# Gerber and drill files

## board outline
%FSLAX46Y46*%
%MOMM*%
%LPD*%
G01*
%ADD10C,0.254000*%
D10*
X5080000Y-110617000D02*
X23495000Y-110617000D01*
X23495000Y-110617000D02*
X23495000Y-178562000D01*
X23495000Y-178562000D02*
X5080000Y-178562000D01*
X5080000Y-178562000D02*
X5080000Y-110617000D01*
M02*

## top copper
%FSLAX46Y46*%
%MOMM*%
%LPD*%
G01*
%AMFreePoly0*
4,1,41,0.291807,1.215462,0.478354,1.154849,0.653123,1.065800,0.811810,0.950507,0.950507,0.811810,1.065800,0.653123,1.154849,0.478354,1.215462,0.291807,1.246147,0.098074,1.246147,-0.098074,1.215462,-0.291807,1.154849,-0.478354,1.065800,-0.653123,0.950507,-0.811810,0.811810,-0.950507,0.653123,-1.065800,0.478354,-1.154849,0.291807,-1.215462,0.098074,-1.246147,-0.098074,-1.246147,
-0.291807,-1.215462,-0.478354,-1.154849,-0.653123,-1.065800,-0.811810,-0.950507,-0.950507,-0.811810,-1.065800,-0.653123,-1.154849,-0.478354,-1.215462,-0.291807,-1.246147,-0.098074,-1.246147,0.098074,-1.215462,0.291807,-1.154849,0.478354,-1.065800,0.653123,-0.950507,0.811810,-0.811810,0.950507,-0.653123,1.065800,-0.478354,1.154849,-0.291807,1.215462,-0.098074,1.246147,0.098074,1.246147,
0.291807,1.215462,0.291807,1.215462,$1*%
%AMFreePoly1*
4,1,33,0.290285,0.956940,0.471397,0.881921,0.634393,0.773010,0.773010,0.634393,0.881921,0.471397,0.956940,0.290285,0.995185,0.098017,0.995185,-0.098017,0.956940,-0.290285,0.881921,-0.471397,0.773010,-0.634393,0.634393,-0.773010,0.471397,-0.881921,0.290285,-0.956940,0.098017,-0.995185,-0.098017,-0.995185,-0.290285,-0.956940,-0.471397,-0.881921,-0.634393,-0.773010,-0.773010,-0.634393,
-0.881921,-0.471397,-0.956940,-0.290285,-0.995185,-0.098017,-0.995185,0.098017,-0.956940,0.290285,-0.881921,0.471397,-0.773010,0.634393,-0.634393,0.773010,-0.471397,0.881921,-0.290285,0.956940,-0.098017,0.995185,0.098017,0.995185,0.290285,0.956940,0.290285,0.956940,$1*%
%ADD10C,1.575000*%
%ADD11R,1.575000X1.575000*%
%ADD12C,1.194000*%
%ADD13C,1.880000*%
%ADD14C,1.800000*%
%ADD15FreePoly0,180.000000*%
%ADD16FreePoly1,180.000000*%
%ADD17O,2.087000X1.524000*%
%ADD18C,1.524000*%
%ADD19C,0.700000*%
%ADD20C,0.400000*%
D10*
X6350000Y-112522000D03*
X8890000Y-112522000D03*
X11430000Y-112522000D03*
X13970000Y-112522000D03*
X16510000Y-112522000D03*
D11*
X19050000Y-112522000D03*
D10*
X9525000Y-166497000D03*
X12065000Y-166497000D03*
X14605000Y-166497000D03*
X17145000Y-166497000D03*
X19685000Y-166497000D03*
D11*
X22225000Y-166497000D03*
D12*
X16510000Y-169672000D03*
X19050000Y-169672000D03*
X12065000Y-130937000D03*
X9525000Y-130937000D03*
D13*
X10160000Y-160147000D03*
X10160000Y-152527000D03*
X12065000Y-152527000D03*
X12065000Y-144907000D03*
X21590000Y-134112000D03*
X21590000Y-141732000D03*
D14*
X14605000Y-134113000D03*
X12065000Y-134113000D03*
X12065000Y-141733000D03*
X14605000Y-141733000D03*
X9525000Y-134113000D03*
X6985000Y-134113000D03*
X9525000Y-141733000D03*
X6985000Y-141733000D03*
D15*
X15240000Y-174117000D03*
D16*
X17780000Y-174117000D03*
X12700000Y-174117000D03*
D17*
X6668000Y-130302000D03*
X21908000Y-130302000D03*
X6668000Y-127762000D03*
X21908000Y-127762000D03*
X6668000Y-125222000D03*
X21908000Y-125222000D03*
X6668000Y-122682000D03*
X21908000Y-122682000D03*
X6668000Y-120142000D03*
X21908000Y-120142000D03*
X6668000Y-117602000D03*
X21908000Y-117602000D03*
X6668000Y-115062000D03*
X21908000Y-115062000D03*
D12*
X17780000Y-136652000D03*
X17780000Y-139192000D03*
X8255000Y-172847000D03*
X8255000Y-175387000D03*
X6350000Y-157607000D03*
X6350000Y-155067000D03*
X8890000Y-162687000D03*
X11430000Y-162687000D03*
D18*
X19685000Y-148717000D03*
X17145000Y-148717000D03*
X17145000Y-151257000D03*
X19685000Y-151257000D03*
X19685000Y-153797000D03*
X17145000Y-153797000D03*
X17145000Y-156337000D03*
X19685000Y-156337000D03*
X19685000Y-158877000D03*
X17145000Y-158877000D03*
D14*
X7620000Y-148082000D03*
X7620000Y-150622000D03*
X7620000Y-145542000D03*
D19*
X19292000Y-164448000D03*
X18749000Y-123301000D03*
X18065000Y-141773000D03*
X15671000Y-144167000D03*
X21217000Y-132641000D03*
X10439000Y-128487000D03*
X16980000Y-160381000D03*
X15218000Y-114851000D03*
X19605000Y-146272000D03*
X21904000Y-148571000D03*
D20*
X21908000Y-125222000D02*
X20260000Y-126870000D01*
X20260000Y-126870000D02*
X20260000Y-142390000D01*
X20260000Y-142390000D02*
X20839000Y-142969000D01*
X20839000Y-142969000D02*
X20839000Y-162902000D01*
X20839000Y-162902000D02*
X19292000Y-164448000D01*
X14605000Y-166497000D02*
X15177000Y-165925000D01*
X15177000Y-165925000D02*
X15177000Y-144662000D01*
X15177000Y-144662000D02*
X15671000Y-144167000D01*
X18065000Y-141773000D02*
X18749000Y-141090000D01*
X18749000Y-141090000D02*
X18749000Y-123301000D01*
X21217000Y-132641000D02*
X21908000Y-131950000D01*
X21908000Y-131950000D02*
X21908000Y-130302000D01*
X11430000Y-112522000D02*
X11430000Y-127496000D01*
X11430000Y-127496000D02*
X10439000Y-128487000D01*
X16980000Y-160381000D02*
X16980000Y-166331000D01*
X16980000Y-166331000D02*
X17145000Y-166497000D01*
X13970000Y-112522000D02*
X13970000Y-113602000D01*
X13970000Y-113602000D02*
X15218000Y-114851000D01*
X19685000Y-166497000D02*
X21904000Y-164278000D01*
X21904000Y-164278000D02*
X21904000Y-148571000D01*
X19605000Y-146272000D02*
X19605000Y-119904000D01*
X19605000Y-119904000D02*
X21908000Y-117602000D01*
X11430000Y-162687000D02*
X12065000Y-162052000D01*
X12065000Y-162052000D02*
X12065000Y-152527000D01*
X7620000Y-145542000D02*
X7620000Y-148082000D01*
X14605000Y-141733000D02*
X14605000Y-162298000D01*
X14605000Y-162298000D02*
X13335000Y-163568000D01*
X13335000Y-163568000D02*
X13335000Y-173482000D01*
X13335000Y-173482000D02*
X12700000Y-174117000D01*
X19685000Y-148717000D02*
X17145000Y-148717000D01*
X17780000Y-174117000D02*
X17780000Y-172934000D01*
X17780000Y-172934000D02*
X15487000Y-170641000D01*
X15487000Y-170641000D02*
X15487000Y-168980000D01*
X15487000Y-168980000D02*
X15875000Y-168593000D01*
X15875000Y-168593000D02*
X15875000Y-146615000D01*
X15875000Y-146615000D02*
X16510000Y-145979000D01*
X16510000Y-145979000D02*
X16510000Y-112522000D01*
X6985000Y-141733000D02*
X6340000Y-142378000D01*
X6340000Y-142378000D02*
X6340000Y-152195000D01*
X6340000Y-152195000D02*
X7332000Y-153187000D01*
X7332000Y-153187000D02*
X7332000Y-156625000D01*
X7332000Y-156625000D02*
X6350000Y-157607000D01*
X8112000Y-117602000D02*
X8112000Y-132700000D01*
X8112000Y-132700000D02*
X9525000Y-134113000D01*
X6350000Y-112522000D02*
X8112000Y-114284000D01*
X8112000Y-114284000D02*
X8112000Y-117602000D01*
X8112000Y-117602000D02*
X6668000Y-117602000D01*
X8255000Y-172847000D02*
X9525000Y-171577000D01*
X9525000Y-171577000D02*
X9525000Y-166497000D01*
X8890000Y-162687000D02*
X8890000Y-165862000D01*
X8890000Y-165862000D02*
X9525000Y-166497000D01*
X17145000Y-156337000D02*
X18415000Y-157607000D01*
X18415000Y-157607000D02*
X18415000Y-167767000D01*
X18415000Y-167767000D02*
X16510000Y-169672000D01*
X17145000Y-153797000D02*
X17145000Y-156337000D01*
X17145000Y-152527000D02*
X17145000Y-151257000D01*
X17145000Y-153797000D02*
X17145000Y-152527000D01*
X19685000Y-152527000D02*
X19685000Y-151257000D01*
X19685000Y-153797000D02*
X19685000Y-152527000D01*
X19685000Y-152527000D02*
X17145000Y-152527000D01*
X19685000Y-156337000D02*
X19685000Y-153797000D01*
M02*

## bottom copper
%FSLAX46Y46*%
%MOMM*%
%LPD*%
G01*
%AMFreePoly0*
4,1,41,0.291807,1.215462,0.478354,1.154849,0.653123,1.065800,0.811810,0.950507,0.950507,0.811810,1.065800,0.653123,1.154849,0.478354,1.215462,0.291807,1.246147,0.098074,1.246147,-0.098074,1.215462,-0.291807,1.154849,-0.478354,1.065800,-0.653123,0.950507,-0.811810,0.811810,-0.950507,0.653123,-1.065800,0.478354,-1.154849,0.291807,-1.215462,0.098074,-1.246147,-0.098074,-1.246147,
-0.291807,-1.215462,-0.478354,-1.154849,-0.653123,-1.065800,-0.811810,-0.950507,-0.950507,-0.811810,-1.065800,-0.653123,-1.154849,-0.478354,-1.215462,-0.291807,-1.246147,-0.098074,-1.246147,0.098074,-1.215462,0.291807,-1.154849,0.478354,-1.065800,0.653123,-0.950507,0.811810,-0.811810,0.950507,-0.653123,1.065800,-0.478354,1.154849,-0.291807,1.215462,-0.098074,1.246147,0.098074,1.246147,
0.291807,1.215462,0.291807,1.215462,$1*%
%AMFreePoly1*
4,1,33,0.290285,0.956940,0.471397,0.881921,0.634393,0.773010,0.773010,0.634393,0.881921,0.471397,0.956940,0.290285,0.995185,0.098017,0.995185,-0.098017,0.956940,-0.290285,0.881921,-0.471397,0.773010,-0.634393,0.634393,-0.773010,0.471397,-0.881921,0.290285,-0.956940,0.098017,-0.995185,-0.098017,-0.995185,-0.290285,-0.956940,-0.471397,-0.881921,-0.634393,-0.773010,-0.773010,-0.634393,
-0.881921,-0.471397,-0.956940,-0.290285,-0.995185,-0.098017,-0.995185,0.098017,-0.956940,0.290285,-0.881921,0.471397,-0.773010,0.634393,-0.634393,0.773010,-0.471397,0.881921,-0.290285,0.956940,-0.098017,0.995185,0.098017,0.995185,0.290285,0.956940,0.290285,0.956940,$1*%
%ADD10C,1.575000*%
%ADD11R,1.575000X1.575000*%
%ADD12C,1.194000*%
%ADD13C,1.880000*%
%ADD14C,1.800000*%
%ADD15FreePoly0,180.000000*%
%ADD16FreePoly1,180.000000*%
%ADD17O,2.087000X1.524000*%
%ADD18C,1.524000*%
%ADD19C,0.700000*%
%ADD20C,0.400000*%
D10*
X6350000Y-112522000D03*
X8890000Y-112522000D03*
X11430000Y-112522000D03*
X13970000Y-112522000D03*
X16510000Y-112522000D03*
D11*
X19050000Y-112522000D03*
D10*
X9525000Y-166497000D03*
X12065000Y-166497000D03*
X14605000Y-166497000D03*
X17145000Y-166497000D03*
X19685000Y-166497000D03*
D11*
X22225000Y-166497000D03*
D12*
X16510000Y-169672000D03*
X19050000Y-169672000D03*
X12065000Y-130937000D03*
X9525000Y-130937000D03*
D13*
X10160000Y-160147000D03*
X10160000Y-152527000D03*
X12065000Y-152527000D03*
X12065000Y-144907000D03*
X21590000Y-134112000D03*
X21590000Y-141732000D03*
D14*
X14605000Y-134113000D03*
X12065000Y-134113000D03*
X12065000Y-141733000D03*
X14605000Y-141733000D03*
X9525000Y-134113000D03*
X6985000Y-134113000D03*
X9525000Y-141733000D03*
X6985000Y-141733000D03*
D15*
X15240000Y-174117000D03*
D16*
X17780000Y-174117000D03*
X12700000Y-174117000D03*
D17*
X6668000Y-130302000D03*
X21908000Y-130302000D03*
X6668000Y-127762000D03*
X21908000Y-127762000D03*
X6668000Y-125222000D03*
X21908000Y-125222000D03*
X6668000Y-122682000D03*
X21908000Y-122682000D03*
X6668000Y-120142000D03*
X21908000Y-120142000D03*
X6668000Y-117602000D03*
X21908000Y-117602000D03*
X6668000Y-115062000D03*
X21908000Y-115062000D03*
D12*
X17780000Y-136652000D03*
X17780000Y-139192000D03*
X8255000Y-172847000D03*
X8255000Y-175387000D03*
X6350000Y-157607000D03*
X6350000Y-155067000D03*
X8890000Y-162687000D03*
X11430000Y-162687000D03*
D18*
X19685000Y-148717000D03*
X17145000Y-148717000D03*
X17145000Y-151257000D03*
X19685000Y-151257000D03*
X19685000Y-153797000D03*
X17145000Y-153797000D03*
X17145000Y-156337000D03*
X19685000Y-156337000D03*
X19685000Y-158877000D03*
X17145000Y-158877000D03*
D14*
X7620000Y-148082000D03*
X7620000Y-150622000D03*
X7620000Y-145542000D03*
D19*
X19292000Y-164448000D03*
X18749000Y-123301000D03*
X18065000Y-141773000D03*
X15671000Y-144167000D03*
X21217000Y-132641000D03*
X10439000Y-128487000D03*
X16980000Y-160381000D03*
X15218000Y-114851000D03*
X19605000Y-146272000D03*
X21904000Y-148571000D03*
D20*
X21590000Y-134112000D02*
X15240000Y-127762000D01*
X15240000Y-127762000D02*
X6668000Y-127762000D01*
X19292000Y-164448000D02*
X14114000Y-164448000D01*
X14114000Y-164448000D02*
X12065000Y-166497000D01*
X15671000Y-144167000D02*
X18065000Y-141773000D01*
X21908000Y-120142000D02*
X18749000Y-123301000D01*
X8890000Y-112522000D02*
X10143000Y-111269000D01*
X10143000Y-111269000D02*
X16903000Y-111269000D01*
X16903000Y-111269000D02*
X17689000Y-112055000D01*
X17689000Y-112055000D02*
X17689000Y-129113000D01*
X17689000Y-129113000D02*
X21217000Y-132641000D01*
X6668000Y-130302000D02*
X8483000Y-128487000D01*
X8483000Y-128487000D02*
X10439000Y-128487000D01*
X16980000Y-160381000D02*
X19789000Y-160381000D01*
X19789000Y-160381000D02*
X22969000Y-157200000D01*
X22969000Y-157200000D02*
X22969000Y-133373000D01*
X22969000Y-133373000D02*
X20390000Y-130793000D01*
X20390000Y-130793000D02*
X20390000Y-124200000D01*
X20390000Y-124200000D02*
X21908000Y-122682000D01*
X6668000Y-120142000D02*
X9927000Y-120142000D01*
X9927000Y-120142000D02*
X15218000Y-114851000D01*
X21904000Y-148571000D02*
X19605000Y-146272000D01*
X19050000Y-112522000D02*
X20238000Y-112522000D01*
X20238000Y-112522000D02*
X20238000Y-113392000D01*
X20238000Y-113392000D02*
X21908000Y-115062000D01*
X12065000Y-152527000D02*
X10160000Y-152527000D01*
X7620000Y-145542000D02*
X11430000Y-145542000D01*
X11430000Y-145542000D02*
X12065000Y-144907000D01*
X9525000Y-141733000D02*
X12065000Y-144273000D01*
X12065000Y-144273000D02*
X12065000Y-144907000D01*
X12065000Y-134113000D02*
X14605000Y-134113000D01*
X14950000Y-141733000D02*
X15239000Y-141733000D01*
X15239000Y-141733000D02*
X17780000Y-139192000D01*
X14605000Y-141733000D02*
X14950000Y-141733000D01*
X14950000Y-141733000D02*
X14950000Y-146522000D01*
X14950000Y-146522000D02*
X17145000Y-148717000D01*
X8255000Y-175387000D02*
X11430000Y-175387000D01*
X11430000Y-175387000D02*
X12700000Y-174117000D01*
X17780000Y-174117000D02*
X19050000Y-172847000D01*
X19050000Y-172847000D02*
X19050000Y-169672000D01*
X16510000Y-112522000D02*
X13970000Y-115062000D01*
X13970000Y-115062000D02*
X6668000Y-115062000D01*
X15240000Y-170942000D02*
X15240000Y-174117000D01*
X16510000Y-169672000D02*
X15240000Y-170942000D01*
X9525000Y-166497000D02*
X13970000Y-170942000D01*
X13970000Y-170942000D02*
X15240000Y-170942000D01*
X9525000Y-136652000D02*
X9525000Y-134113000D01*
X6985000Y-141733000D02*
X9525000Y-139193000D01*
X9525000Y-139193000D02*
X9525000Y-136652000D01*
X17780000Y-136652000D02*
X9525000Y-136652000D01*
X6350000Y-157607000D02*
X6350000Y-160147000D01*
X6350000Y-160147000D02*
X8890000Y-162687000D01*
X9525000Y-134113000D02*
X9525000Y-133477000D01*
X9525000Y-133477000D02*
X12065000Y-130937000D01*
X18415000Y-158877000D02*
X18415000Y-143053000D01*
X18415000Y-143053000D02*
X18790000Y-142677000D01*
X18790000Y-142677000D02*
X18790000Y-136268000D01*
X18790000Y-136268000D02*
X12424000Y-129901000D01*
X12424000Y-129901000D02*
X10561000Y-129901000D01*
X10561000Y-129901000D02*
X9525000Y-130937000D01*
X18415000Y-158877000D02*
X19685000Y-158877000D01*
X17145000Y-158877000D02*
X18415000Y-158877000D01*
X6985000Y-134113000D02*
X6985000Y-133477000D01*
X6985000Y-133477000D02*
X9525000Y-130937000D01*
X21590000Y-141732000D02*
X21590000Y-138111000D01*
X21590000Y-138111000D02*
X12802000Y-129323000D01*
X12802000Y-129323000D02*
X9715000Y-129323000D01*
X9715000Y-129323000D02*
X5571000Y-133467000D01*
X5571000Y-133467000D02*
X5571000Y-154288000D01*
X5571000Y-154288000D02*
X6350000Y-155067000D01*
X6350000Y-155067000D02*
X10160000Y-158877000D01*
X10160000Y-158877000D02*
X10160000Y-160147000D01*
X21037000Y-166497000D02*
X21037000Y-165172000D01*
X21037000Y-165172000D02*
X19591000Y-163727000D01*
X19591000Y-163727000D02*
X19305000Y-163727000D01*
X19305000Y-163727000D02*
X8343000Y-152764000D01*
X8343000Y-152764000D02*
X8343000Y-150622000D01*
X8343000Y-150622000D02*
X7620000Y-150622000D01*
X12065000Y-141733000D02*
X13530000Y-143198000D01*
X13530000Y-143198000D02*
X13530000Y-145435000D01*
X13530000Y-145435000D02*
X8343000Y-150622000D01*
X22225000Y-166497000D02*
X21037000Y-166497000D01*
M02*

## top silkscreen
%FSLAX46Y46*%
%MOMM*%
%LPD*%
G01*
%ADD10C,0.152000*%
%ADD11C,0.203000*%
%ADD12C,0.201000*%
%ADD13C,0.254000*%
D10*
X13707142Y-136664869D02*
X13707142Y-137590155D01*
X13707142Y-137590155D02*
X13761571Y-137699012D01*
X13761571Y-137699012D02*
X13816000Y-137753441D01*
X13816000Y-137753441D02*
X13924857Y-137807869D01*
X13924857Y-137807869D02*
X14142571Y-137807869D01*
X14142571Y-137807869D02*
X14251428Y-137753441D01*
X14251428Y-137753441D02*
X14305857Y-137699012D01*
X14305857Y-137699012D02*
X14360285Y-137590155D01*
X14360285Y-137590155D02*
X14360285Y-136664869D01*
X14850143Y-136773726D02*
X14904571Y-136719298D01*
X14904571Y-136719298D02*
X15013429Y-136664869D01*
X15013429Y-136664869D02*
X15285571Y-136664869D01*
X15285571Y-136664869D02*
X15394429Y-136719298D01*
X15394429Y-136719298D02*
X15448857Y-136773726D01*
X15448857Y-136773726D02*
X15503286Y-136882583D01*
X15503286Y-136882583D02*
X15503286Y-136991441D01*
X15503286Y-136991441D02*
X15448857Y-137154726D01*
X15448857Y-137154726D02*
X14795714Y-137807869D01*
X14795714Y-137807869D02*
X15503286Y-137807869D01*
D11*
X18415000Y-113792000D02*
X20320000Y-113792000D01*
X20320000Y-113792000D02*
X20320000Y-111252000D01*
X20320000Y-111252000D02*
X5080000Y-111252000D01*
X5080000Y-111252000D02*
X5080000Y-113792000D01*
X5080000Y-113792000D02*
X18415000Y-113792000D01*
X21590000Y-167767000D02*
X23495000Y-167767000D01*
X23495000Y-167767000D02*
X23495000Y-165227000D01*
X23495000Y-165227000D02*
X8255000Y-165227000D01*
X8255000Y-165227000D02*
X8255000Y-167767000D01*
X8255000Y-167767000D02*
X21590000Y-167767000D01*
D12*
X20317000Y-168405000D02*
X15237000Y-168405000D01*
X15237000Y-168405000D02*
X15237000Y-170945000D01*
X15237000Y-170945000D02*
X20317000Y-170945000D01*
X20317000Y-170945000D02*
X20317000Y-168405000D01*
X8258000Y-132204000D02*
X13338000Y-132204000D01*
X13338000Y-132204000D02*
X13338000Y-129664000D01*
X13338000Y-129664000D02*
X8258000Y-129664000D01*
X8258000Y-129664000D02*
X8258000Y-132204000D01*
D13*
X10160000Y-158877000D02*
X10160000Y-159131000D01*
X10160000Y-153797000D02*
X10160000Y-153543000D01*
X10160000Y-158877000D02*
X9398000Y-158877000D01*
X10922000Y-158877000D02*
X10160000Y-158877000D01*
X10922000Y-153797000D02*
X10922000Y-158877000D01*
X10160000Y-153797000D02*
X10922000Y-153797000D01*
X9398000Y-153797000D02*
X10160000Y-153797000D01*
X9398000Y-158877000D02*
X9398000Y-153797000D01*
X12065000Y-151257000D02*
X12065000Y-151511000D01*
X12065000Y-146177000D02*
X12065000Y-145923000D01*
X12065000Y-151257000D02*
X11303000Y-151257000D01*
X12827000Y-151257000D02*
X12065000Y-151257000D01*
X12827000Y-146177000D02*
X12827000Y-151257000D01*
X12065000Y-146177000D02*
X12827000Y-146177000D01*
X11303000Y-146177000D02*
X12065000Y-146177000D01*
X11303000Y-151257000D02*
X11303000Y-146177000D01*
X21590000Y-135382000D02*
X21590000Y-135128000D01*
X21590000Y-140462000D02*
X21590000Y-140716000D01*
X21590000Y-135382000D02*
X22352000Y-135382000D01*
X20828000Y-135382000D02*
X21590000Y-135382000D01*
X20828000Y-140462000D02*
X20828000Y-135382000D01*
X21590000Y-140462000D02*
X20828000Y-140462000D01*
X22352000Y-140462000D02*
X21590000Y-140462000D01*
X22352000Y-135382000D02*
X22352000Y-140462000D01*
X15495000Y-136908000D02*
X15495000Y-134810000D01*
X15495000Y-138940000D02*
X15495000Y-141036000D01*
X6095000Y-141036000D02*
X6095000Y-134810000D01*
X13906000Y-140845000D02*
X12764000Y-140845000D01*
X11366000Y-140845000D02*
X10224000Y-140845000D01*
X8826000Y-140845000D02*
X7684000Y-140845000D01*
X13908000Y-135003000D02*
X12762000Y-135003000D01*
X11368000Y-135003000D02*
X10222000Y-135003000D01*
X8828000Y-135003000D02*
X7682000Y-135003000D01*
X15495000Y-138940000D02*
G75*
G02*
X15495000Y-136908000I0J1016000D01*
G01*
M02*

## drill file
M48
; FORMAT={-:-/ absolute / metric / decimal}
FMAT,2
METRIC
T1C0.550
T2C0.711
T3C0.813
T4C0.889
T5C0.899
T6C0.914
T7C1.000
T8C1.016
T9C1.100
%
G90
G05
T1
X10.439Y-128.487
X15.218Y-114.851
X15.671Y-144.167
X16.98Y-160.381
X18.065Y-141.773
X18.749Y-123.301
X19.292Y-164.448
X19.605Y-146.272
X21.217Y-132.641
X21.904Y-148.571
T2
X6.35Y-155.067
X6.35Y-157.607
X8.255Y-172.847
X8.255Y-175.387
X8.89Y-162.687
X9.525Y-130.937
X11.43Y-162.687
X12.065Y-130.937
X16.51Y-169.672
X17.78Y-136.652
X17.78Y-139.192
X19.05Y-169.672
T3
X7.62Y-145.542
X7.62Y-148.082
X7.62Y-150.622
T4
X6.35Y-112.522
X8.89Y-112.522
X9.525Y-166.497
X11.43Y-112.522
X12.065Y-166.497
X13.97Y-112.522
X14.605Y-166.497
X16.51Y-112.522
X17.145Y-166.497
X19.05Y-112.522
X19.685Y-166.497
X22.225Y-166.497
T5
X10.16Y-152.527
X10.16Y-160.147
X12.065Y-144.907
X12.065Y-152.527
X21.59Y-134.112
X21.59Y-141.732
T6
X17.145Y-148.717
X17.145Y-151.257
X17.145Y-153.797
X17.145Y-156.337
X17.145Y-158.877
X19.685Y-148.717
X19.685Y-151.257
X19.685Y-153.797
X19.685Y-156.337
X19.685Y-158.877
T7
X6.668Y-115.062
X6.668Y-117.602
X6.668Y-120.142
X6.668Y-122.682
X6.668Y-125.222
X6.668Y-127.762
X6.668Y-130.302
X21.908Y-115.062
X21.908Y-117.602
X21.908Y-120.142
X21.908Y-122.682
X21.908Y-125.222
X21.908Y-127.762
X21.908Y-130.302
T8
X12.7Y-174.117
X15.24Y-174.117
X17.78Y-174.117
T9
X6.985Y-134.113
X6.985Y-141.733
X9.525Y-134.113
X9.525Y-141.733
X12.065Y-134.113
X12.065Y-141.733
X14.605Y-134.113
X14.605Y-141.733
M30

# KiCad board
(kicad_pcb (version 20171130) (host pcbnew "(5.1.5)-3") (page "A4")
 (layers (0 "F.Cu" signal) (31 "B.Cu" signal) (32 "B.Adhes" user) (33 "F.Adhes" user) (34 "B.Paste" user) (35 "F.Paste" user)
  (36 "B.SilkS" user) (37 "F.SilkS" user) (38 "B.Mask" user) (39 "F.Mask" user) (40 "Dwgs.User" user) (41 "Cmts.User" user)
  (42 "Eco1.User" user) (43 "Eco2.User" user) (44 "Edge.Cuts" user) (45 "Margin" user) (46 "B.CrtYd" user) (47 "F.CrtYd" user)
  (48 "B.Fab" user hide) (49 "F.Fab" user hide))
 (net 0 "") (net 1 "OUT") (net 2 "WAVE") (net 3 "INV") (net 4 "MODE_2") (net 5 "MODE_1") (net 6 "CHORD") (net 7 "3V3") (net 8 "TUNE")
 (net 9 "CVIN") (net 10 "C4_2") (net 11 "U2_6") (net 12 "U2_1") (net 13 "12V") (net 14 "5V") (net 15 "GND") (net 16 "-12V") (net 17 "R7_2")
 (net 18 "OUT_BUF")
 (segment (start 21.59 134.112) (end 15.24 127.762) (width 0.4) (layer "B.Cu") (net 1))
 (segment (start 15.24 127.762) (end 6.668 127.762) (width 0.4) (layer "B.Cu") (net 1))
 (segment (start 19.292 164.448) (end 14.114 164.448) (width 0.4) (layer "B.Cu") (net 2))
 (segment (start 14.114 164.448) (end 12.065 166.497) (width 0.4) (layer "B.Cu") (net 2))
 (segment (start 15.671 144.167) (end 18.065 141.773) (width 0.4) (layer "B.Cu") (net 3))
 (segment (start 21.908 120.142) (end 18.749 123.301) (width 0.4) (layer "B.Cu") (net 3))
 (segment (start 8.89 112.522) (end 10.143 111.269) (width 0.4) (layer "B.Cu") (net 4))
 (segment (start 10.143 111.269) (end 16.903 111.269) (width 0.4) (layer "B.Cu") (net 4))
 (segment (start 16.903 111.269) (end 17.689 112.055) (width 0.4) (layer "B.Cu") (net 4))
 (segment (start 17.689 112.055) (end 17.689 129.113) (width 0.4) (layer "B.Cu") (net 4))
 (segment (start 17.689 129.113) (end 21.217 132.641) (width 0.4) (layer "B.Cu") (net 4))
 (segment (start 6.668 130.302) (end 8.483 128.487) (width 0.4) (layer "B.Cu") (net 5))
 (segment (start 8.483 128.487) (end 10.439 128.487) (width 0.4) (layer "B.Cu") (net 5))
 (segment (start 16.98 160.381) (end 19.789 160.381) (width 0.4) (layer "B.Cu") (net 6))
 (segment (start 19.789 160.381) (end 22.969 157.2) (width 0.4) (layer "B.Cu") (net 6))
 (segment (start 22.969 157.2) (end 22.969 133.373) (width 0.4) (layer "B.Cu") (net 6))
 (segment (start 22.969 133.373) (end 20.39 130.793) (width 0.4) (layer "B.Cu") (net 6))
 (segment (start 20.39 130.793) (end 20.39 124.2) (width 0.4) (layer "B.Cu") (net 6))
 (segment (start 20.39 124.2) (end 21.908 122.682) (width 0.4) (layer "B.Cu") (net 6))
 (segment (start 6.668 120.142) (end 9.927 120.142) (width 0.4) (layer "B.Cu") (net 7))
 (segment (start 9.927 120.142) (end 15.218 114.851) (width 0.4) (layer "B.Cu") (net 7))
 (segment (start 21.904 148.571) (end 19.605 146.272) (width 0.4) (layer "B.Cu") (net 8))
 (segment (start 19.05 112.522) (end 20.238 112.522) (width 0.4) (layer "B.Cu") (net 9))
 (segment (start 20.238 112.522) (end 20.238 113.392) (width 0.4) (layer "B.Cu") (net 9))
 (segment (start 20.238 113.392) (end 21.908 115.062) (width 0.4) (layer "B.Cu") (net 9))
 (segment (start 12.065 152.527) (end 10.16 152.527) (width 0.4) (layer "B.Cu") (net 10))
 (segment (start 7.62 145.542) (end 11.43 145.542) (width 0.4) (layer "B.Cu") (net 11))
 (segment (start 11.43 145.542) (end 12.065 144.907) (width 0.4) (layer "B.Cu") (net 11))
 (segment (start 9.525 141.733) (end 12.065 144.273) (width 0.4) (layer "B.Cu") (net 11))
 (segment (start 12.065 144.273) (end 12.065 144.907) (width 0.4) (layer "B.Cu") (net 11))
 (segment (start 12.065 134.113) (end 14.605 134.113) (width 0.4) (layer "B.Cu") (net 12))
 (segment (start 14.95 141.733) (end 15.239 141.733) (width 0.4) (layer "B.Cu") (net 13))
 (segment (start 15.239 141.733) (end 17.78 139.192) (width 0.4) (layer "B.Cu") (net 13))
 (segment (start 14.605 141.733) (end 14.95 141.733) (width 0.4) (layer "B.Cu") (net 13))
 (segment (start 14.95 141.733) (end 14.95 146.522) (width 0.4) (layer "B.Cu") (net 13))
 (segment (start 14.95 146.522) (end 17.145 148.717) (width 0.4) (layer "B.Cu") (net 13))
 (segment (start 8.255 175.387) (end 11.43 175.387) (width 0.4) (layer "B.Cu") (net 13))
 (segment (start 11.43 175.387) (end 12.7 174.117) (width 0.4) (layer "B.Cu") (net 13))
 (segment (start 17.78 174.117) (end 19.05 172.847) (width 0.4) (layer "B.Cu") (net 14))
 (segment (start 19.05 172.847) (end 19.05 169.672) (width 0.4) (layer "B.Cu") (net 14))
 (segment (start 16.51 112.522) (end 13.97 115.062) (width 0.4) (layer "B.Cu") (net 14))
 (segment (start 13.97 115.062) (end 6.668 115.062) (width 0.4) (layer "B.Cu") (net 14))
 (segment (start 15.24 170.942) (end 15.24 174.117) (width 0.4) (layer "B.Cu") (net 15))
 (segment (start 16.51 169.672) (end 15.24 170.942) (width 0.4) (layer "B.Cu") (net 15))
 (segment (start 9.525 166.497) (end 13.97 170.942) (width 0.4) (layer "B.Cu") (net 15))
 (segment (start 13.97 170.942) (end 15.24 170.942) (width 0.4) (layer "B.Cu") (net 15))
 (segment (start 9.525 136.652) (end 9.525 134.113) (width 0.4) (layer "B.Cu") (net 15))
 (segment (start 6.985 141.733) (end 9.525 139.193) (width 0.4) (layer "B.Cu") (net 15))
 (segment (start 9.525 139.193) (end 9.525 136.652) (width 0.4) (layer "B.Cu") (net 15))
 (segment (start 17.78 136.652) (end 9.525 136.652) (width 0.4) (layer "B.Cu") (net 15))
 (segment (start 6.35 157.607) (end 6.35 160.147) (width 0.4) (layer "B.Cu") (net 15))
 (segment (start 6.35 160.147) (end 8.89 162.687) (width 0.4) (layer "B.Cu") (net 15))
 (segment (start 9.525 134.113) (end 9.525 133.477) (width 0.4) (layer "B.Cu") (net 15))
 (segment (start 9.525 133.477) (end 12.065 130.937) (width 0.4) (layer "B.Cu") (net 15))
 (segment (start 18.415 158.877) (end 18.415 143.053) (width 0.4) (layer "B.Cu") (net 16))
 (segment (start 18.415 143.053) (end 18.79 142.677) (width 0.4) (layer "B.Cu") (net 16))
 (segment (start 18.79 142.677) (end 18.79 136.268) (width 0.4) (layer "B.Cu") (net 16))
 (segment (start 18.79 136.268) (end 12.424 129.901) (width 0.4) (layer "B.Cu") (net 16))
 (segment (start 12.424 129.901) (end 10.561 129.901) (width 0.4) (layer "B.Cu") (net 16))
 (segment (start 10.561 129.901) (end 9.525 130.937) (width 0.4) (layer "B.Cu") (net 16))
 (segment (start 18.415 158.877) (end 19.685 158.877) (width 0.4) (layer "B.Cu") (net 16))
 (segment (start 17.145 158.877) (end 18.415 158.877) (width 0.4) (layer "B.Cu") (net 16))
 (segment (start 6.985 134.113) (end 6.985 133.477) (width 0.4) (layer "B.Cu") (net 16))
 (segment (start 6.985 133.477) (end 9.525 130.937) (width 0.4) (layer "B.Cu") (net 16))
 (segment (start 21.59 141.732) (end 21.59 138.111) (width 0.4) (layer "B.Cu") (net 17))
 (segment (start 21.59 138.111) (end 12.802 129.323) (width 0.4) (layer "B.Cu") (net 17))
 (segment (start 12.802 129.323) (end 9.715 129.323) (width 0.4) (layer "B.Cu") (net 17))
 (segment (start 9.715 129.323) (end 5.571 133.467) (width 0.4) (layer "B.Cu") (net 17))
 (segment (start 5.571 133.467) (end 5.571 154.288) (width 0.4) (layer "B.Cu") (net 17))
 (segment (start 5.571 154.288) (end 6.35 155.067) (width 0.4) (layer "B.Cu") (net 17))
 (segment (start 6.35 155.067) (end 10.16 158.877) (width 0.4) (layer "B.Cu") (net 17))
 (segment (start 10.16 158.877) (end 10.16 160.147) (width 0.4) (layer "B.Cu") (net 17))
 (segment (start 21.037 166.497) (end 21.037 165.172) (width 0.4) (layer "B.Cu") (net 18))
 (segment (start 21.037 165.172) (end 19.591 163.727) (width 0.4) (layer "B.Cu") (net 18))
 (segment (start 19.591 163.727) (end 19.305 163.727) (width 0.4) (layer "B.Cu") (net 18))
 (segment (start 19.305 163.727) (end 8.343 152.764) (width 0.4) (layer "B.Cu") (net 18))
 (segment (start 8.343 152.764) (end 8.343 150.622) (width 0.4) (layer "B.Cu") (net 18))
 (segment (start 8.343 150.622) (end 7.62 150.622) (width 0.4) (layer "B.Cu") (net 18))
 (segment (start 12.065 141.733) (end 13.53 143.198) (width 0.4) (layer "B.Cu") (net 18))
 (segment (start 13.53 143.198) (end 13.53 145.435) (width 0.4) (layer "B.Cu") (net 18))
 (segment (start 13.53 145.435) (end 8.343 150.622) (width 0.4) (layer "B.Cu") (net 18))
 (segment (start 22.225 166.497) (end 21.037 166.497) (width 0.4) (layer "B.Cu") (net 18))
 (gr_line (start 5.08 110.617) (end 23.495 110.617) (width 0.254) (layer "Edge.Cuts"))
 (gr_line (start 23.495 110.617) (end 23.495 178.562) (width 0.254) (layer "Edge.Cuts"))
 (gr_line (start 23.495 178.562) (end 5.08 178.562) (width 0.254) (layer "Edge.Cuts"))
 (gr_line (start 5.08 178.562) (end 5.08 110.617) (width 0.254) (layer "Edge.Cuts"))
 (segment (start 21.908 125.222) (end 20.26 126.87) (width 0.4) (layer "F.Cu") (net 2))
 (segment (start 20.26 126.87) (end 20.26 142.39) (width 0.4) (layer "F.Cu") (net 2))
 (segment (start 20.26 142.39) (end 20.839 142.969) (width 0.4) (layer "F.Cu") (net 2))
 (segment (start 20.839 142.969) (end 20.839 162.902) (width 0.4) (layer "F.Cu") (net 2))
 (segment (start 20.839 162.902) (end 19.292 164.448) (width 0.4) (layer "F.Cu") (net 2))
 (segment (start 14.605 166.497) (end 15.177 165.925) (width 0.4) (layer "F.Cu") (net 3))
 (segment (start 15.177 165.925) (end 15.177 144.662) (width 0.4) (layer "F.Cu") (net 3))
 (segment (start 15.177 144.662) (end 15.671 144.167) (width 0.4) (layer "F.Cu") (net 3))
 (segment (start 18.065 141.773) (end 18.749 141.09) (width 0.4) (layer "F.Cu") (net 3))
 (segment (start 18.749 141.09) (end 18.749 123.301) (width 0.4) (layer "F.Cu") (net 3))
 (segment (start 21.217 132.641) (end 21.908 131.95) (width 0.4) (layer "F.Cu") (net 4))
 (segment (start 21.908 131.95) (end 21.908 130.302) (width 0.4) (layer "F.Cu") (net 4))
 (segment (start 11.43 112.522) (end 11.43 127.496) (width 0.4) (layer "F.Cu") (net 5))
 (segment (start 11.43 127.496) (end 10.439 128.487) (width 0.4) (layer "F.Cu") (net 5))
 (segment (start 16.98 160.381) (end 16.98 166.331) (width 0.4) (layer "F.Cu") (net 6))
 (segment (start 16.98 166.331) (end 17.145 166.497) (width 0.4) (layer "F.Cu") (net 6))
 (segment (start 13.97 112.522) (end 13.97 113.602) (width 0.4) (layer "F.Cu") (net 7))
 (segment (start 13.97 113.602) (end 15.218 114.851) (width 0.4) (layer "F.Cu") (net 7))
 (segment (start 19.685 166.497) (end 21.904 164.278) (width 0.4) (layer "F.Cu") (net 8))
 (segment (start 21.904 164.278) (end 21.904 148.571) (width 0.4) (layer "F.Cu") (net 8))
 (segment (start 19.605 146.272) (end 19.605 119.904) (width 0.4) (layer "F.Cu") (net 8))
 (segment (start 19.605 119.904) (end 21.908 117.602) (width 0.4) (layer "F.Cu") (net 8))
 (segment (start 11.43 162.687) (end 12.065 162.052) (width 0.4) (layer "F.Cu") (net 10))
 (segment (start 12.065 162.052) (end 12.065 152.527) (width 0.4) (layer "F.Cu") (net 10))
 (segment (start 7.62 145.542) (end 7.62 148.082) (width 0.4) (layer "F.Cu") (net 11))
 (segment (start 14.605 141.733) (end 14.605 162.298) (width 0.4) (layer "F.Cu") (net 13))
 (segment (start 14.605 162.298) (end 13.335 163.568) (width 0.4) (layer "F.Cu") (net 13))
 (segment (start 13.335 163.568) (end 13.335 173.482) (width 0.4) (layer "F.Cu") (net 13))
 (segment (start 13.335 173.482) (end 12.7 174.117) (width 0.4) (layer "F.Cu") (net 13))
 (segment (start 19.685 148.717) (end 17.145 148.717) (width 0.4) (layer "F.Cu") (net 13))
 (segment (start 17.78 174.117) (end 17.78 172.934) (width 0.4) (layer "F.Cu") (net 14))
 (segment (start 17.78 172.934) (end 15.487 170.641) (width 0.4) (layer "F.Cu") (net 14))
 (segment (start 15.487 170.641) (end 15.487 168.98) (width 0.4) (layer "F.Cu") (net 14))
 (segment (start 15.487 168.98) (end 15.875 168.593) (width 0.4) (layer "F.Cu") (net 14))
 (segment (start 15.875 168.593) (end 15.875 146.615) (width 0.4) (layer "F.Cu") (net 14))
 (segment (start 15.875 146.615) (end 16.51 145.979) (width 0.4) (layer "F.Cu") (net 14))
 (segment (start 16.51 145.979) (end 16.51 112.522) (width 0.4) (layer "F.Cu") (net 14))
 (segment (start 6.985 141.733) (end 6.34 142.378) (width 0.4) (layer "F.Cu") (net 15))
 (segment (start 6.34 142.378) (end 6.34 152.195) (width 0.4) (layer "F.Cu") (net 15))
 (segment (start 6.34 152.195) (end 7.332 153.187) (width 0.4) (layer "F.Cu") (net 15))
 (segment (start 7.332 153.187) (end 7.332 156.625) (width 0.4) (layer "F.Cu") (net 15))
 (segment (start 7.332 156.625) (end 6.35 157.607) (width 0.4) (layer "F.Cu") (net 15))
 (segment (start 8.112 117.602) (end 8.112 132.7) (width 0.4) (layer "F.Cu") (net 15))
 (segment (start 8.112 132.7) (end 9.525 134.113) (width 0.4) (layer "F.Cu") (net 15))
 (segment (start 6.35 112.522) (end 8.112 114.284) (width 0.4) (layer "F.Cu") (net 15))
 (segment (start 8.112 114.284) (end 8.112 117.602) (width 0.4) (layer "F.Cu") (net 15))
 (segment (start 8.112 117.602) (end 6.668 117.602) (width 0.4) (layer "F.Cu") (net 15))
 (segment (start 8.255 172.847) (end 9.525 171.577) (width 0.4) (layer "F.Cu") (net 15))
 (segment (start 9.525 171.577) (end 9.525 166.497) (width 0.4) (layer "F.Cu") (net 15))
 (segment (start 8.89 162.687) (end 8.89 165.862) (width 0.4) (layer "F.Cu") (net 15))
 (segment (start 8.89 165.862) (end 9.525 166.497) (width 0.4) (layer "F.Cu") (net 15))
 (segment (start 17.145 156.337) (end 18.415 157.607) (width 0.4) (layer "F.Cu") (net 15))
 (segment (start 18.415 157.607) (end 18.415 167.767) (width 0.4) (layer "F.Cu") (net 15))
 (segment (start 18.415 167.767) (end 16.51 169.672) (width 0.4) (layer "F.Cu") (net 15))
 (segment (start 17.145 153.797) (end 17.145 156.337) (width 0.4) (layer "F.Cu") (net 15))
 (segment (start 17.145 152.527) (end 17.145 151.257) (width 0.4) (layer "F.Cu") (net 15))
 (segment (start 17.145 153.797) (end 17.145 152.527) (width 0.4) (layer "F.Cu") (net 15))
 (segment (start 19.685 152.527) (end 19.685 151.257) (width 0.4) (layer "F.Cu") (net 15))
 (segment (start 19.685 153.797) (end 19.685 152.527) (width 0.4) (layer "F.Cu") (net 15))
 (segment (start 19.685 152.527) (end 17.145 152.527) (width 0.4) (layer "F.Cu") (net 15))
 (segment (start 19.685 156.337) (end 19.685 153.797) (width 0.4) (layer "F.Cu") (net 15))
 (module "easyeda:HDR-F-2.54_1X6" (layer "F.Cu") (at 13.97 112.522 180)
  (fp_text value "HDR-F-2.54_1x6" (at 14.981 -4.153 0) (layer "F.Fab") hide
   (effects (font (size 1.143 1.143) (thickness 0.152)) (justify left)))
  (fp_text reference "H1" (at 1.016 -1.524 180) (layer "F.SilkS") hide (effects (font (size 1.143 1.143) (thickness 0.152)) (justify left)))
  (fp_line (start -4.445 -1.27) (end -6.35 -1.27) (width 0.203) (layer "F.SilkS"))
  (fp_line (start -6.35 -1.27) (end -6.35 1.27) (width 0.203) (layer "F.SilkS"))
  (fp_line (start -6.35 1.27) (end 8.89 1.27) (width 0.203) (layer "F.SilkS"))
  (fp_line (start 8.89 1.27) (end 8.89 -1.27) (width 0.203) (layer "F.SilkS"))
  (fp_line (start 8.89 -1.27) (end -4.445 -1.27) (width 0.203) (layer "F.SilkS"))
  (pad 6 thru_hole circle (at 7.62 0 180) (size 1.575 1.575) (layers "*.Cu" "*.Paste" "*.Mask") (drill 0.889) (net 15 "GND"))
  (pad 5 thru_hole circle (at 5.08 0 180) (size 1.575 1.575) (layers "*.Cu" "*.Paste" "*.Mask") (drill 0.889) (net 4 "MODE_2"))
  (pad 4 thru_hole circle (at 2.54 0 180) (size 1.575 1.575) (layers "*.Cu" "*.Paste" "*.Mask") (drill 0.889) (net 5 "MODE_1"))
  (pad 3 thru_hole circle (at 0 0 180) (size 1.575 1.575) (layers "*.Cu" "*.Paste" "*.Mask") (drill 0.889) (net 7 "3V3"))
  (pad 2 thru_hole circle (at -2.54 0 180) (size 1.575 1.575) (layers "*.Cu" "*.Paste" "*.Mask") (drill 0.889) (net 14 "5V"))
  (pad 1 thru_hole rect (at -5.08 0 180) (size 1.575 1.575) (layers "*.Cu" "*.Paste" "*.Mask") (drill 0.889) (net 9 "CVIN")))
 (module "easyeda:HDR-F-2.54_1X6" (layer "F.Cu") (at 17.145 166.497 180)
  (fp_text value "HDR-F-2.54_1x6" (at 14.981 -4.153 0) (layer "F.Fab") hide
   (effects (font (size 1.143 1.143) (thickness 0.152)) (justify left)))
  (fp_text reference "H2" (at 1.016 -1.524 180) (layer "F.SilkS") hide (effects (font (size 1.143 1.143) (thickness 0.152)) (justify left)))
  (fp_line (start -4.445 -1.27) (end -6.35 -1.27) (width 0.203) (layer "F.SilkS"))
  (fp_line (start -6.35 -1.27) (end -6.35 1.27) (width 0.203) (layer "F.SilkS"))
  (fp_line (start -6.35 1.27) (end 8.89 1.27) (width 0.203) (layer "F.SilkS"))
  (fp_line (start 8.89 1.27) (end 8.89 -1.27) (width 0.203) (layer "F.SilkS"))
  (fp_line (start 8.89 -1.27) (end -4.445 -1.27) (width 0.203) (layer "F.SilkS"))
  (pad 6 thru_hole circle (at 7.62 0 180) (size 1.575 1.575) (layers "*.Cu" "*.Paste" "*.Mask") (drill 0.889) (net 15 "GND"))
  (pad 5 thru_hole circle (at 5.08 0 180) (size 1.575 1.575) (layers "*.Cu" "*.Paste" "*.Mask") (drill 0.889) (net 2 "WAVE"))
  (pad 4 thru_hole circle (at 2.54 0 180) (size 1.575 1.575) (layers "*.Cu" "*.Paste" "*.Mask") (drill 0.889) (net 3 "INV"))
  (pad 3 thru_hole circle (at 0 0 180) (size 1.575 1.575) (layers "*.Cu" "*.Paste" "*.Mask") (drill 0.889) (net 6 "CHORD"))
  (pad 2 thru_hole circle (at -2.54 0 180) (size 1.575 1.575) (layers "*.Cu" "*.Paste" "*.Mask") (drill 0.889) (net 8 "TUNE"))
  (pad 1 thru_hole rect (at -5.08 0 180) (size 1.575 1.575) (layers "*.Cu" "*.Paste" "*.Mask") (drill 0.889) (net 18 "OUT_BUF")))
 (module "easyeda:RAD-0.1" (layer "F.Cu") (at 17.78 169.672)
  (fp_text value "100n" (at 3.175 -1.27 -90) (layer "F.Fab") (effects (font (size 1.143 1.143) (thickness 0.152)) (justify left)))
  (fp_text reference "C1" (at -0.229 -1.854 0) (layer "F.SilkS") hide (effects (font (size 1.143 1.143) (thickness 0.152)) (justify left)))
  (fp_line (start 2.537 -1.267) (end -2.543 -1.267) (width 0.201) (layer "F.SilkS"))
  (fp_line (start -2.543 -1.267) (end -2.543 1.273) (width 0.201) (layer "F.SilkS"))
  (fp_line (start -2.543 1.273) (end 2.537 1.273) (width 0.201) (layer "F.SilkS"))
  (fp_line (start 2.537 1.273) (end 2.537 -1.267) (width 0.201) (layer "F.SilkS"))
  (pad 1 thru_hole circle (at -1.27 0 0) (size 1.194 1.194) (layers "*.Cu" "*.Paste" "*.Mask") (drill 0.711) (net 15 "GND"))
  (pad 2 thru_hole circle (at 1.27 0 0) (size 1.194 1.194) (layers "*.Cu" "*.Paste" "*.Mask") (drill 0.711) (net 14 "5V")))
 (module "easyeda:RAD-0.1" (layer "F.Cu") (at 10.795 130.937 180)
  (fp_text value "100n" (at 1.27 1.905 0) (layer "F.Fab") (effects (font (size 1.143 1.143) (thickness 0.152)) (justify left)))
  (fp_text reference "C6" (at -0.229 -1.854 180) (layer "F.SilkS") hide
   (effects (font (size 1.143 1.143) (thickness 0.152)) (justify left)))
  (fp_line (start 2.537 -1.267) (end -2.543 -1.267) (width 0.201) (layer "F.SilkS"))
  (fp_line (start -2.543 -1.267) (end -2.543 1.273) (width 0.201) (layer "F.SilkS"))
  (fp_line (start -2.543 1.273) (end 2.537 1.273) (width 0.201) (layer "F.SilkS"))
  (fp_line (start 2.537 1.273) (end 2.537 -1.267) (width 0.201) (layer "F.SilkS"))
  (pad 1 thru_hole circle (at -1.27 0 180) (size 1.194 1.194) (layers "*.Cu" "*.Paste" "*.Mask") (drill 0.711) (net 15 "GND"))
  (pad 2 thru_hole circle (at 1.27 0 180) (size 1.194 1.194) (layers "*.Cu" "*.Paste" "*.Mask") (drill 0.711) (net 16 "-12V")))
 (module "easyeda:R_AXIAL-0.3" (layer "F.Cu") (at 10.16 156.337 90)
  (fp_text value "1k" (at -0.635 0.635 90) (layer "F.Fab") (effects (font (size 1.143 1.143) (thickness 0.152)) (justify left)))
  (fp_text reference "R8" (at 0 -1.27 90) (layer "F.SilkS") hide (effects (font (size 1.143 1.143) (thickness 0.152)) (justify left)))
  (fp_line (start -2.54 0) (end -2.794 0) (width 0.254) (layer "F.SilkS"))
  (fp_line (start 2.54 0) (end 2.794 0) (width 0.254) (layer "F.SilkS"))
  (fp_line (start -2.54 0) (end -2.54 -0.762) (width 0.254) (layer "F.SilkS"))
  (fp_line (start -2.54 0.762) (end -2.54 0) (width 0.254) (layer "F.SilkS"))
  (fp_line (start 2.54 0.762) (end -2.54 0.762) (width 0.254) (layer "F.SilkS"))
  (fp_line (start 2.54 0) (end 2.54 0.762) (width 0.254) (layer "F.SilkS"))
  (fp_line (start 2.54 -0.762) (end 2.54 0) (width 0.254) (layer "F.SilkS"))
  (fp_line (start -2.54 -0.762) (end 2.54 -0.762) (width 0.254) (layer "F.SilkS"))
  (pad 1 thru_hole circle (at -3.81 0 90) (size 1.88 1.88) (layers "*.Cu" "*.Paste" "*.Mask") (drill 0.899) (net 17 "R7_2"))
  (pad 2 thru_hole circle (at 3.81 0 90) (size 1.88 1.88) (layers "*.Cu" "*.Paste" "*.Mask") (drill 0.899) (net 10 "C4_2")))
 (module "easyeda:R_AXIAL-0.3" (layer "F.Cu") (at 12.065 148.717 90)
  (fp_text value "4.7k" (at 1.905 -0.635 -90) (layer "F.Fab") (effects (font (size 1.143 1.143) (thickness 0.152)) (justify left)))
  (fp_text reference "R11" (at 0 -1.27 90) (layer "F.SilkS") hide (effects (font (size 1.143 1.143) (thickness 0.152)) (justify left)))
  (fp_line (start -2.54 0) (end -2.794 0) (width 0.254) (layer "F.SilkS"))
  (fp_line (start 2.54 0) (end 2.794 0) (width 0.254) (layer "F.SilkS"))
  (fp_line (start -2.54 0) (end -2.54 -0.762) (width 0.254) (layer "F.SilkS"))
  (fp_line (start -2.54 0.762) (end -2.54 0) (width 0.254) (layer "F.SilkS"))
  (fp_line (start 2.54 0.762) (end -2.54 0.762) (width 0.254) (layer "F.SilkS"))
  (fp_line (start 2.54 0) (end 2.54 0.762) (width 0.254) (layer "F.SilkS"))
  (fp_line (start 2.54 -0.762) (end 2.54 0) (width 0.254) (layer "F.SilkS"))
  (fp_line (start -2.54 -0.762) (end 2.54 -0.762) (width 0.254) (layer "F.SilkS"))
  (pad 1 thru_hole circle (at -3.81 0 90) (size 1.88 1.88) (layers "*.Cu" "*.Paste" "*.Mask") (drill 0.899) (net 10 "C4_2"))
  (pad 2 thru_hole circle (at 3.81 0 90) (size 1.88 1.88) (layers "*.Cu" "*.Paste" "*.Mask") (drill 0.899) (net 11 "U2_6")))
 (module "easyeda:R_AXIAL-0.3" (layer "F.Cu") (at 21.59 137.922 -90)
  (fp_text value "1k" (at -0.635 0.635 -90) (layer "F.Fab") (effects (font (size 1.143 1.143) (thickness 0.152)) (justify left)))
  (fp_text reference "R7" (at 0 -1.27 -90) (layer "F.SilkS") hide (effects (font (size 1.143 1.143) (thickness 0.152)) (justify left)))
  (fp_line (start -2.54 0) (end -2.794 0) (width 0.254) (layer "F.SilkS"))
  (fp_line (start 2.54 0) (end 2.794 0) (width 0.254) (layer "F.SilkS"))
  (fp_line (start -2.54 0) (end -2.54 -0.762) (width 0.254) (layer "F.SilkS"))
  (fp_line (start -2.54 0.762) (end -2.54 0) (width 0.254) (layer "F.SilkS"))
  (fp_line (start 2.54 0.762) (end -2.54 0.762) (width 0.254) (layer "F.SilkS"))
  (fp_line (start 2.54 0) (end 2.54 0.762) (width 0.254) (layer "F.SilkS"))
  (fp_line (start 2.54 -0.762) (end 2.54 0) (width 0.254) (layer "F.SilkS"))
  (fp_line (start -2.54 -0.762) (end 2.54 -0.762) (width 0.254) (layer "F.SilkS"))
  (pad 1 thru_hole circle (at -3.81 0 -90) (size 1.88 1.88) (layers "*.Cu" "*.Paste" "*.Mask") (drill 0.899) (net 1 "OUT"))
  (pad 2 thru_hole circle (at 3.81 0 -90) (size 1.88 1.88) (layers "*.Cu" "*.Paste" "*.Mask") (drill 0.899) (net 17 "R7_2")))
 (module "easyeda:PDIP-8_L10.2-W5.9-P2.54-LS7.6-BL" (layer "F.Cu") (at 10.795 137.923 180)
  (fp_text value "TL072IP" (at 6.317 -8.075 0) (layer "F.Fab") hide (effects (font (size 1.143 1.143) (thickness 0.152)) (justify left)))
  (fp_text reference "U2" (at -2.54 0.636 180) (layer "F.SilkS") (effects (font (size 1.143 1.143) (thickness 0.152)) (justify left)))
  (fp_line (start -4.7 1.015) (end -4.7 3.113) (width 0.254) (layer "F.SilkS"))
  (fp_line (start -4.7 -1.017) (end -4.7 -3.113) (width 0.254) (layer "F.SilkS"))
  (fp_line (start 4.7 -3.113) (end 4.7 3.113) (width 0.254) (layer "F.SilkS"))
  (fp_line (start -3.111 -2.922) (end -1.969 -2.922) (width 0.254) (layer "F.SilkS"))
  (fp_line (start -0.571 -2.922) (end 0.571 -2.922) (width 0.254) (layer "F.SilkS"))
  (fp_line (start 1.969 -2.922) (end 3.111 -2.922) (width 0.254) (layer "F.SilkS"))
  (fp_line (start -3.113 2.92) (end -1.967 2.92) (width 0.254) (layer "F.SilkS"))
  (fp_line (start -0.573 2.92) (end 0.573 2.92) (width 0.254) (layer "F.SilkS"))
  (fp_line (start 1.967 2.92) (end 3.113 2.92) (width 0.254) (layer "F.SilkS"))
  (fp_arc (start -4.7 -0.001) (end -4.7 -1.017) (angle 180) (width 0.254) (layer "F.SilkS"))
  (pad 1 thru_hole circle (at -3.81 3.81 -90) (size 1.8 1.8) (layers "*.Cu" "*.Paste" "*.Mask") (drill 1.1) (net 12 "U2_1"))
  (pad 2 thru_hole circle (at -1.27 3.81 -90) (size 1.8 1.8) (layers "*.Cu" "*.Paste" "*.Mask") (drill 1.1) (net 12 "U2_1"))
  (pad 7 thru_hole circle (at -1.27 -3.81 -90) (size 1.8 1.8) (layers "*.Cu" "*.Paste" "*.Mask") (drill 1.1) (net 18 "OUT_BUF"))
  (pad 8 thru_hole circle (at -3.81 -3.81 -90) (size 1.8 1.8) (layers "*.Cu" "*.Paste" "*.Mask") (drill 1.1) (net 13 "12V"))
  (pad 3 thru_hole circle (at 1.27 3.81 -90) (size 1.8 1.8) (layers "*.Cu" "*.Paste" "*.Mask") (drill 1.1) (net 15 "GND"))
  (pad 4 thru_hole circle (at 3.81 3.81 -90) (size 1.8 1.8) (layers "*.Cu" "*.Paste" "*.Mask") (drill 1.1) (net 16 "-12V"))
  (pad 6 thru_hole circle (at 1.27 -3.81 -90) (size 1.8 1.8) (layers "*.Cu" "*.Paste" "*.Mask") (drill 1.1) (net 11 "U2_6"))
  (pad 5 thru_hole circle (at 3.81 -3.81 -90) (size 1.8 1.8) (layers "*.Cu" "*.Paste" "*.Mask") (drill 1.1) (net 15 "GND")))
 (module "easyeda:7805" (layer "F.Cu") (at 10.16 176.657 180)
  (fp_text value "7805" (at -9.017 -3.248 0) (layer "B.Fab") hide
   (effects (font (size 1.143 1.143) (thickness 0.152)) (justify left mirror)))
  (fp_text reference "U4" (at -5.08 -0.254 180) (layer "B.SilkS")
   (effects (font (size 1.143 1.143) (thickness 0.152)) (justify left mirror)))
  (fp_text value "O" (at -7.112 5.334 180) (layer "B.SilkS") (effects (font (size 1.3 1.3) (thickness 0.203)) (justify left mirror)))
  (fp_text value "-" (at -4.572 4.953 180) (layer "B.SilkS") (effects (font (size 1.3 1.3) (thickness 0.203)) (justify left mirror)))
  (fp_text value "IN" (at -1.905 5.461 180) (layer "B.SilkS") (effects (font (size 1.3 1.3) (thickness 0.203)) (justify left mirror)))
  (pad 2 thru_hole custom (at -5.08 2.54 180) (size 2.5 3.5) (layers "*.Cu" "*.Paste" "*.Mask") (drill 1.016) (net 15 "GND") (primitives))
  (pad 3 thru_hole custom (at -7.62 2.54 180) (size 2 3.5) (layers "*.Cu" "*.Paste" "*.Mask") (drill 1.016) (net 14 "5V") (primitives))
  (pad 1 thru_hole custom (at -2.54 2.54 180) (size 2 3.5) (layers "*.Cu" "*.Paste" "*.Mask") (drill 1.016) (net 13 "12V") (primitives)))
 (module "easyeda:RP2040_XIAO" (layer "F.Cu") (at 14.288 122.682 -90)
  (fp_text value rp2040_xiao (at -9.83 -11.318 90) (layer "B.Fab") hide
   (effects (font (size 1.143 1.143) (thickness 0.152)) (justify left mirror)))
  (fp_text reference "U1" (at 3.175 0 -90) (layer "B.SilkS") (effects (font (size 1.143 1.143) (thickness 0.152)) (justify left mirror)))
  (pad 1 thru_hole oval (at 7.62 7.62 -90) (size 1.524 2.087) (layers "*.Cu" "*.Paste" "*.Mask") (drill 1) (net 5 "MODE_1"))
  (pad 14 thru_hole oval (at 7.62 -7.62 -90) (size 1.524 2.087) (layers "*.Cu" "*.Paste" "*.Mask") (drill 1) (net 4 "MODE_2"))
  (pad 2 thru_hole oval (at 5.08 7.62 -90) (size 1.524 2.087) (layers "*.Cu" "*.Paste" "*.Mask") (drill 1) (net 1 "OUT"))
  (pad 13 thru_hole oval (at 5.08 -7.62 -90) (size 1.524 2.087) (layers "*.Cu" "*.Paste" "*.Mask") (drill 1))
  (pad 3 thru_hole oval (at 2.54 7.62 -90) (size 1.524 2.087) (layers "*.Cu" "*.Paste" "*.Mask") (drill 1))
  (pad 12 thru_hole oval (at 2.54 -7.62 -90) (size 1.524 2.087) (layers "*.Cu" "*.Paste" "*.Mask") (drill 1) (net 2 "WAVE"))
  (pad 4 thru_hole oval (at 0 7.62 -90) (size 1.524 2.087) (layers "*.Cu" "*.Paste" "*.Mask") (drill 1))
  (pad 11 thru_hole oval (at 0 -7.62 -90) (size 1.524 2.087) (layers "*.Cu" "*.Paste" "*.Mask") (drill 1) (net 6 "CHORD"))
  (pad 5 thru_hole oval (at -2.54 7.62 -90) (size 1.524 2.087) (layers "*.Cu" "*.Paste" "*.Mask") (drill 1) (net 7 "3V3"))
  (pad 10 thru_hole oval (at -2.54 -7.62 -90) (size 1.524 2.087) (layers "*.Cu" "*.Paste" "*.Mask") (drill 1) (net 3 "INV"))
  (pad 6 thru_hole oval (at -5.08 7.62 -90) (size 1.524 2.087) (layers "*.Cu" "*.Paste" "*.Mask") (drill 1) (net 15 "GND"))
  (pad 9 thru_hole oval (at -5.08 -7.62 -90) (size 1.524 2.087) (layers "*.Cu" "*.Paste" "*.Mask") (drill 1) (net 8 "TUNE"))
  (pad 7 thru_hole oval (at -7.62 7.62 -90) (size 1.524 2.087) (layers "*.Cu" "*.Paste" "*.Mask") (drill 1) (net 14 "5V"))
  (pad 8 thru_hole oval (at -7.62 -7.62 -90) (size 1.524 2.087) (layers "*.Cu" "*.Paste" "*.Mask") (drill 1) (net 9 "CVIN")))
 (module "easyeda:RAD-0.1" (layer "F.Cu") (at 17.78 137.922 90)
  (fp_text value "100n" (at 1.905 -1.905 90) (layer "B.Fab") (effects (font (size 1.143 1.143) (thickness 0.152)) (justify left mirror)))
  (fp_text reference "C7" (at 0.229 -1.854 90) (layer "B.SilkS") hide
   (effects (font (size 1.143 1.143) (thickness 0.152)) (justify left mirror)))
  (pad 1 thru_hole circle (at 1.27 0 90) (size 1.194 1.194) (layers "*.Cu" "*.Paste" "*.Mask") (drill 0.711) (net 15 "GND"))
  (pad 2 thru_hole circle (at -1.27 0 90) (size 1.194 1.194) (layers "*.Cu" "*.Paste" "*.Mask") (drill 0.711) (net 13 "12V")))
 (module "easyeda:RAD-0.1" (layer "F.Cu") (at 8.255 174.117 90)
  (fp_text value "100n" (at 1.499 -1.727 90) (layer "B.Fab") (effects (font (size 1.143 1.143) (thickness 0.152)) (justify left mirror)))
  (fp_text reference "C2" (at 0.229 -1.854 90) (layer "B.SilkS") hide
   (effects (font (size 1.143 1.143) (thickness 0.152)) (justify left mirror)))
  (pad 1 thru_hole circle (at 1.27 0 90) (size 1.194 1.194) (layers "*.Cu" "*.Paste" "*.Mask") (drill 0.711) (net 15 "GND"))
  (pad 2 thru_hole circle (at -1.27 0 90) (size 1.194 1.194) (layers "*.Cu" "*.Paste" "*.Mask") (drill 0.711) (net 13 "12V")))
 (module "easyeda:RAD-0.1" (layer "F.Cu") (at 6.35 156.337 -90)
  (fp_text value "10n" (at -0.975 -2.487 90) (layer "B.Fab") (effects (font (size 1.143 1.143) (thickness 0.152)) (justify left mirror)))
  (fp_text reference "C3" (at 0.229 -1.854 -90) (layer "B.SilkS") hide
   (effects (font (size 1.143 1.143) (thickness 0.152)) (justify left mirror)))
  (pad 1 thru_hole circle (at 1.27 0 -90) (size 1.194 1.194) (layers "*.Cu" "*.Paste" "*.Mask") (drill 0.711) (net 15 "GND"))
  (pad 2 thru_hole circle (at -1.27 0 -90) (size 1.194 1.194) (layers "*.Cu" "*.Paste" "*.Mask") (drill 0.711) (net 17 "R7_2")))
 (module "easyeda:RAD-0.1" (layer "F.Cu") (at 10.16 162.687 180)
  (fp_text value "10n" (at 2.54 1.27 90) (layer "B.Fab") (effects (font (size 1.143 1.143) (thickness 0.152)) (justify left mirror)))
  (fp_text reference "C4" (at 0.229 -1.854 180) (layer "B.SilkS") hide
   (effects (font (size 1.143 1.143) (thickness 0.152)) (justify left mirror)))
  (pad 1 thru_hole circle (at 1.27 0 180) (size 1.194 1.194) (layers "*.Cu" "*.Paste" "*.Mask") (drill 0.711) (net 15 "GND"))
  (pad 2 thru_hole circle (at -1.27 0 180) (size 1.194 1.194) (layers "*.Cu" "*.Paste" "*.Mask") (drill 0.711) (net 10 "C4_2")))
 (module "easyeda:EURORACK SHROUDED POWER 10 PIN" (layer "F.Cu") (at 18.415 153.797)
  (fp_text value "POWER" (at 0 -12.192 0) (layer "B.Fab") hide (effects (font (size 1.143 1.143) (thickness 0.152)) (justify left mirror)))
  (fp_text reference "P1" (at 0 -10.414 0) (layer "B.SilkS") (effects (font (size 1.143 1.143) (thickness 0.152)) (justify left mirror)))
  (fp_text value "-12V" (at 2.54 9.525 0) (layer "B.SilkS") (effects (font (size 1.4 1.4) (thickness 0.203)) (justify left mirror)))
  (pad 1 thru_hole circle (at 1.27 -5.08 0) (size 1.524 1.524) (layers "*.Cu" "*.Paste" "*.Mask") (drill 0.914) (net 13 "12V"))
  (pad 1 thru_hole circle (at -1.27 -5.08 0) (size 1.524 1.524) (layers "*.Cu" "*.Paste" "*.Mask") (drill 0.914) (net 13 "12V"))
  (pad 2 thru_hole circle (at -1.27 -2.54 0) (size 1.524 1.524) (layers "*.Cu" "*.Paste" "*.Mask") (drill 0.914) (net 15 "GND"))
  (pad 2 thru_hole circle (at 1.27 -2.54 0) (size 1.524 1.524) (layers "*.Cu" "*.Paste" "*.Mask") (drill 0.914) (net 15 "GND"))
  (pad 3 thru_hole circle (at 1.27 0 0) (size 1.524 1.524) (layers "*.Cu" "*.Paste" "*.Mask") (drill 0.914) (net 15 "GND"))
  (pad 3 thru_hole circle (at -1.27 0 0) (size 1.524 1.524) (layers "*.Cu" "*.Paste" "*.Mask") (drill 0.914) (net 15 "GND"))
  (pad 4 thru_hole circle (at -1.27 2.54 0) (size 1.524 1.524) (layers "*.Cu" "*.Paste" "*.Mask") (drill 0.914) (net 15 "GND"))
  (pad 4 thru_hole circle (at 1.27 2.54 0) (size 1.524 1.524) (layers "*.Cu" "*.Paste" "*.Mask") (drill 0.914) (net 15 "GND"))
  (pad 5 thru_hole circle (at 1.27 5.08 0) (size 1.524 1.524) (layers "*.Cu" "*.Paste" "*.Mask") (drill 0.914) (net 16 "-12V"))
  (pad 5 thru_hole circle (at -1.27 5.08 0) (size 1.524 1.524) (layers "*.Cu" "*.Paste" "*.Mask") (drill 0.914) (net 16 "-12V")))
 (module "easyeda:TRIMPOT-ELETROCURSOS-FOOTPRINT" (layer "F.Cu") (at 7.62 148.082 180)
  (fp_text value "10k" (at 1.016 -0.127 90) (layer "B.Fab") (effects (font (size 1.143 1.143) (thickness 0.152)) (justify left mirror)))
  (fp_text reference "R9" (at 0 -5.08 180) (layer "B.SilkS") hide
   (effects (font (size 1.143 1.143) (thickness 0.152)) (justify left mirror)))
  (pad 2 thru_hole circle (at 0 0 180) (size 1.8 1.8) (layers "*.Cu" "*.Paste" "*.Mask") (drill 0.813) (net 11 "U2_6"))
  (pad 3 thru_hole circle (at 0 -2.54 180) (size 1.8 1.8) (layers "*.Cu" "*.Paste" "*.Mask") (drill 0.813) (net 18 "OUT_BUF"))
  (pad 1 thru_hole circle (at 0 2.54 180) (size 1.8 1.8) (layers "*.Cu" "*.Paste" "*.Mask") (drill 0.813) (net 11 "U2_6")))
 (via (at 19.292 164.448) (size 0.7) (drill 0.55) (layers "F.Cu" "B.Cu") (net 2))
 (via (at 18.749 123.301) (size 0.7) (drill 0.55) (layers "F.Cu" "B.Cu") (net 3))
 (via (at 18.065 141.773) (size 0.7) (drill 0.55) (layers "F.Cu" "B.Cu") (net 3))
 (via (at 15.671 144.167) (size 0.7) (drill 0.55) (layers "F.Cu" "B.Cu") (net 3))
 (via (at 21.217 132.641) (size 0.7) (drill 0.55) (layers "F.Cu" "B.Cu") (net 4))
 (via (at 10.439 128.487) (size 0.7) (drill 0.55) (layers "F.Cu" "B.Cu") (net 5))
 (via (at 16.98 160.381) (size 0.7) (drill 0.55) (layers "F.Cu" "B.Cu") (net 6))
 (via (at 15.218 114.851) (size 0.7) (drill 0.55) (layers "F.Cu" "B.Cu") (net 7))
 (via (at 19.605 146.272) (size 0.7) (drill 0.55) (layers "F.Cu" "B.Cu") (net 8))
 (via (at 21.904 148.571) (size 0.7) (drill 0.55) (layers "F.Cu" "B.Cu") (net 8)))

